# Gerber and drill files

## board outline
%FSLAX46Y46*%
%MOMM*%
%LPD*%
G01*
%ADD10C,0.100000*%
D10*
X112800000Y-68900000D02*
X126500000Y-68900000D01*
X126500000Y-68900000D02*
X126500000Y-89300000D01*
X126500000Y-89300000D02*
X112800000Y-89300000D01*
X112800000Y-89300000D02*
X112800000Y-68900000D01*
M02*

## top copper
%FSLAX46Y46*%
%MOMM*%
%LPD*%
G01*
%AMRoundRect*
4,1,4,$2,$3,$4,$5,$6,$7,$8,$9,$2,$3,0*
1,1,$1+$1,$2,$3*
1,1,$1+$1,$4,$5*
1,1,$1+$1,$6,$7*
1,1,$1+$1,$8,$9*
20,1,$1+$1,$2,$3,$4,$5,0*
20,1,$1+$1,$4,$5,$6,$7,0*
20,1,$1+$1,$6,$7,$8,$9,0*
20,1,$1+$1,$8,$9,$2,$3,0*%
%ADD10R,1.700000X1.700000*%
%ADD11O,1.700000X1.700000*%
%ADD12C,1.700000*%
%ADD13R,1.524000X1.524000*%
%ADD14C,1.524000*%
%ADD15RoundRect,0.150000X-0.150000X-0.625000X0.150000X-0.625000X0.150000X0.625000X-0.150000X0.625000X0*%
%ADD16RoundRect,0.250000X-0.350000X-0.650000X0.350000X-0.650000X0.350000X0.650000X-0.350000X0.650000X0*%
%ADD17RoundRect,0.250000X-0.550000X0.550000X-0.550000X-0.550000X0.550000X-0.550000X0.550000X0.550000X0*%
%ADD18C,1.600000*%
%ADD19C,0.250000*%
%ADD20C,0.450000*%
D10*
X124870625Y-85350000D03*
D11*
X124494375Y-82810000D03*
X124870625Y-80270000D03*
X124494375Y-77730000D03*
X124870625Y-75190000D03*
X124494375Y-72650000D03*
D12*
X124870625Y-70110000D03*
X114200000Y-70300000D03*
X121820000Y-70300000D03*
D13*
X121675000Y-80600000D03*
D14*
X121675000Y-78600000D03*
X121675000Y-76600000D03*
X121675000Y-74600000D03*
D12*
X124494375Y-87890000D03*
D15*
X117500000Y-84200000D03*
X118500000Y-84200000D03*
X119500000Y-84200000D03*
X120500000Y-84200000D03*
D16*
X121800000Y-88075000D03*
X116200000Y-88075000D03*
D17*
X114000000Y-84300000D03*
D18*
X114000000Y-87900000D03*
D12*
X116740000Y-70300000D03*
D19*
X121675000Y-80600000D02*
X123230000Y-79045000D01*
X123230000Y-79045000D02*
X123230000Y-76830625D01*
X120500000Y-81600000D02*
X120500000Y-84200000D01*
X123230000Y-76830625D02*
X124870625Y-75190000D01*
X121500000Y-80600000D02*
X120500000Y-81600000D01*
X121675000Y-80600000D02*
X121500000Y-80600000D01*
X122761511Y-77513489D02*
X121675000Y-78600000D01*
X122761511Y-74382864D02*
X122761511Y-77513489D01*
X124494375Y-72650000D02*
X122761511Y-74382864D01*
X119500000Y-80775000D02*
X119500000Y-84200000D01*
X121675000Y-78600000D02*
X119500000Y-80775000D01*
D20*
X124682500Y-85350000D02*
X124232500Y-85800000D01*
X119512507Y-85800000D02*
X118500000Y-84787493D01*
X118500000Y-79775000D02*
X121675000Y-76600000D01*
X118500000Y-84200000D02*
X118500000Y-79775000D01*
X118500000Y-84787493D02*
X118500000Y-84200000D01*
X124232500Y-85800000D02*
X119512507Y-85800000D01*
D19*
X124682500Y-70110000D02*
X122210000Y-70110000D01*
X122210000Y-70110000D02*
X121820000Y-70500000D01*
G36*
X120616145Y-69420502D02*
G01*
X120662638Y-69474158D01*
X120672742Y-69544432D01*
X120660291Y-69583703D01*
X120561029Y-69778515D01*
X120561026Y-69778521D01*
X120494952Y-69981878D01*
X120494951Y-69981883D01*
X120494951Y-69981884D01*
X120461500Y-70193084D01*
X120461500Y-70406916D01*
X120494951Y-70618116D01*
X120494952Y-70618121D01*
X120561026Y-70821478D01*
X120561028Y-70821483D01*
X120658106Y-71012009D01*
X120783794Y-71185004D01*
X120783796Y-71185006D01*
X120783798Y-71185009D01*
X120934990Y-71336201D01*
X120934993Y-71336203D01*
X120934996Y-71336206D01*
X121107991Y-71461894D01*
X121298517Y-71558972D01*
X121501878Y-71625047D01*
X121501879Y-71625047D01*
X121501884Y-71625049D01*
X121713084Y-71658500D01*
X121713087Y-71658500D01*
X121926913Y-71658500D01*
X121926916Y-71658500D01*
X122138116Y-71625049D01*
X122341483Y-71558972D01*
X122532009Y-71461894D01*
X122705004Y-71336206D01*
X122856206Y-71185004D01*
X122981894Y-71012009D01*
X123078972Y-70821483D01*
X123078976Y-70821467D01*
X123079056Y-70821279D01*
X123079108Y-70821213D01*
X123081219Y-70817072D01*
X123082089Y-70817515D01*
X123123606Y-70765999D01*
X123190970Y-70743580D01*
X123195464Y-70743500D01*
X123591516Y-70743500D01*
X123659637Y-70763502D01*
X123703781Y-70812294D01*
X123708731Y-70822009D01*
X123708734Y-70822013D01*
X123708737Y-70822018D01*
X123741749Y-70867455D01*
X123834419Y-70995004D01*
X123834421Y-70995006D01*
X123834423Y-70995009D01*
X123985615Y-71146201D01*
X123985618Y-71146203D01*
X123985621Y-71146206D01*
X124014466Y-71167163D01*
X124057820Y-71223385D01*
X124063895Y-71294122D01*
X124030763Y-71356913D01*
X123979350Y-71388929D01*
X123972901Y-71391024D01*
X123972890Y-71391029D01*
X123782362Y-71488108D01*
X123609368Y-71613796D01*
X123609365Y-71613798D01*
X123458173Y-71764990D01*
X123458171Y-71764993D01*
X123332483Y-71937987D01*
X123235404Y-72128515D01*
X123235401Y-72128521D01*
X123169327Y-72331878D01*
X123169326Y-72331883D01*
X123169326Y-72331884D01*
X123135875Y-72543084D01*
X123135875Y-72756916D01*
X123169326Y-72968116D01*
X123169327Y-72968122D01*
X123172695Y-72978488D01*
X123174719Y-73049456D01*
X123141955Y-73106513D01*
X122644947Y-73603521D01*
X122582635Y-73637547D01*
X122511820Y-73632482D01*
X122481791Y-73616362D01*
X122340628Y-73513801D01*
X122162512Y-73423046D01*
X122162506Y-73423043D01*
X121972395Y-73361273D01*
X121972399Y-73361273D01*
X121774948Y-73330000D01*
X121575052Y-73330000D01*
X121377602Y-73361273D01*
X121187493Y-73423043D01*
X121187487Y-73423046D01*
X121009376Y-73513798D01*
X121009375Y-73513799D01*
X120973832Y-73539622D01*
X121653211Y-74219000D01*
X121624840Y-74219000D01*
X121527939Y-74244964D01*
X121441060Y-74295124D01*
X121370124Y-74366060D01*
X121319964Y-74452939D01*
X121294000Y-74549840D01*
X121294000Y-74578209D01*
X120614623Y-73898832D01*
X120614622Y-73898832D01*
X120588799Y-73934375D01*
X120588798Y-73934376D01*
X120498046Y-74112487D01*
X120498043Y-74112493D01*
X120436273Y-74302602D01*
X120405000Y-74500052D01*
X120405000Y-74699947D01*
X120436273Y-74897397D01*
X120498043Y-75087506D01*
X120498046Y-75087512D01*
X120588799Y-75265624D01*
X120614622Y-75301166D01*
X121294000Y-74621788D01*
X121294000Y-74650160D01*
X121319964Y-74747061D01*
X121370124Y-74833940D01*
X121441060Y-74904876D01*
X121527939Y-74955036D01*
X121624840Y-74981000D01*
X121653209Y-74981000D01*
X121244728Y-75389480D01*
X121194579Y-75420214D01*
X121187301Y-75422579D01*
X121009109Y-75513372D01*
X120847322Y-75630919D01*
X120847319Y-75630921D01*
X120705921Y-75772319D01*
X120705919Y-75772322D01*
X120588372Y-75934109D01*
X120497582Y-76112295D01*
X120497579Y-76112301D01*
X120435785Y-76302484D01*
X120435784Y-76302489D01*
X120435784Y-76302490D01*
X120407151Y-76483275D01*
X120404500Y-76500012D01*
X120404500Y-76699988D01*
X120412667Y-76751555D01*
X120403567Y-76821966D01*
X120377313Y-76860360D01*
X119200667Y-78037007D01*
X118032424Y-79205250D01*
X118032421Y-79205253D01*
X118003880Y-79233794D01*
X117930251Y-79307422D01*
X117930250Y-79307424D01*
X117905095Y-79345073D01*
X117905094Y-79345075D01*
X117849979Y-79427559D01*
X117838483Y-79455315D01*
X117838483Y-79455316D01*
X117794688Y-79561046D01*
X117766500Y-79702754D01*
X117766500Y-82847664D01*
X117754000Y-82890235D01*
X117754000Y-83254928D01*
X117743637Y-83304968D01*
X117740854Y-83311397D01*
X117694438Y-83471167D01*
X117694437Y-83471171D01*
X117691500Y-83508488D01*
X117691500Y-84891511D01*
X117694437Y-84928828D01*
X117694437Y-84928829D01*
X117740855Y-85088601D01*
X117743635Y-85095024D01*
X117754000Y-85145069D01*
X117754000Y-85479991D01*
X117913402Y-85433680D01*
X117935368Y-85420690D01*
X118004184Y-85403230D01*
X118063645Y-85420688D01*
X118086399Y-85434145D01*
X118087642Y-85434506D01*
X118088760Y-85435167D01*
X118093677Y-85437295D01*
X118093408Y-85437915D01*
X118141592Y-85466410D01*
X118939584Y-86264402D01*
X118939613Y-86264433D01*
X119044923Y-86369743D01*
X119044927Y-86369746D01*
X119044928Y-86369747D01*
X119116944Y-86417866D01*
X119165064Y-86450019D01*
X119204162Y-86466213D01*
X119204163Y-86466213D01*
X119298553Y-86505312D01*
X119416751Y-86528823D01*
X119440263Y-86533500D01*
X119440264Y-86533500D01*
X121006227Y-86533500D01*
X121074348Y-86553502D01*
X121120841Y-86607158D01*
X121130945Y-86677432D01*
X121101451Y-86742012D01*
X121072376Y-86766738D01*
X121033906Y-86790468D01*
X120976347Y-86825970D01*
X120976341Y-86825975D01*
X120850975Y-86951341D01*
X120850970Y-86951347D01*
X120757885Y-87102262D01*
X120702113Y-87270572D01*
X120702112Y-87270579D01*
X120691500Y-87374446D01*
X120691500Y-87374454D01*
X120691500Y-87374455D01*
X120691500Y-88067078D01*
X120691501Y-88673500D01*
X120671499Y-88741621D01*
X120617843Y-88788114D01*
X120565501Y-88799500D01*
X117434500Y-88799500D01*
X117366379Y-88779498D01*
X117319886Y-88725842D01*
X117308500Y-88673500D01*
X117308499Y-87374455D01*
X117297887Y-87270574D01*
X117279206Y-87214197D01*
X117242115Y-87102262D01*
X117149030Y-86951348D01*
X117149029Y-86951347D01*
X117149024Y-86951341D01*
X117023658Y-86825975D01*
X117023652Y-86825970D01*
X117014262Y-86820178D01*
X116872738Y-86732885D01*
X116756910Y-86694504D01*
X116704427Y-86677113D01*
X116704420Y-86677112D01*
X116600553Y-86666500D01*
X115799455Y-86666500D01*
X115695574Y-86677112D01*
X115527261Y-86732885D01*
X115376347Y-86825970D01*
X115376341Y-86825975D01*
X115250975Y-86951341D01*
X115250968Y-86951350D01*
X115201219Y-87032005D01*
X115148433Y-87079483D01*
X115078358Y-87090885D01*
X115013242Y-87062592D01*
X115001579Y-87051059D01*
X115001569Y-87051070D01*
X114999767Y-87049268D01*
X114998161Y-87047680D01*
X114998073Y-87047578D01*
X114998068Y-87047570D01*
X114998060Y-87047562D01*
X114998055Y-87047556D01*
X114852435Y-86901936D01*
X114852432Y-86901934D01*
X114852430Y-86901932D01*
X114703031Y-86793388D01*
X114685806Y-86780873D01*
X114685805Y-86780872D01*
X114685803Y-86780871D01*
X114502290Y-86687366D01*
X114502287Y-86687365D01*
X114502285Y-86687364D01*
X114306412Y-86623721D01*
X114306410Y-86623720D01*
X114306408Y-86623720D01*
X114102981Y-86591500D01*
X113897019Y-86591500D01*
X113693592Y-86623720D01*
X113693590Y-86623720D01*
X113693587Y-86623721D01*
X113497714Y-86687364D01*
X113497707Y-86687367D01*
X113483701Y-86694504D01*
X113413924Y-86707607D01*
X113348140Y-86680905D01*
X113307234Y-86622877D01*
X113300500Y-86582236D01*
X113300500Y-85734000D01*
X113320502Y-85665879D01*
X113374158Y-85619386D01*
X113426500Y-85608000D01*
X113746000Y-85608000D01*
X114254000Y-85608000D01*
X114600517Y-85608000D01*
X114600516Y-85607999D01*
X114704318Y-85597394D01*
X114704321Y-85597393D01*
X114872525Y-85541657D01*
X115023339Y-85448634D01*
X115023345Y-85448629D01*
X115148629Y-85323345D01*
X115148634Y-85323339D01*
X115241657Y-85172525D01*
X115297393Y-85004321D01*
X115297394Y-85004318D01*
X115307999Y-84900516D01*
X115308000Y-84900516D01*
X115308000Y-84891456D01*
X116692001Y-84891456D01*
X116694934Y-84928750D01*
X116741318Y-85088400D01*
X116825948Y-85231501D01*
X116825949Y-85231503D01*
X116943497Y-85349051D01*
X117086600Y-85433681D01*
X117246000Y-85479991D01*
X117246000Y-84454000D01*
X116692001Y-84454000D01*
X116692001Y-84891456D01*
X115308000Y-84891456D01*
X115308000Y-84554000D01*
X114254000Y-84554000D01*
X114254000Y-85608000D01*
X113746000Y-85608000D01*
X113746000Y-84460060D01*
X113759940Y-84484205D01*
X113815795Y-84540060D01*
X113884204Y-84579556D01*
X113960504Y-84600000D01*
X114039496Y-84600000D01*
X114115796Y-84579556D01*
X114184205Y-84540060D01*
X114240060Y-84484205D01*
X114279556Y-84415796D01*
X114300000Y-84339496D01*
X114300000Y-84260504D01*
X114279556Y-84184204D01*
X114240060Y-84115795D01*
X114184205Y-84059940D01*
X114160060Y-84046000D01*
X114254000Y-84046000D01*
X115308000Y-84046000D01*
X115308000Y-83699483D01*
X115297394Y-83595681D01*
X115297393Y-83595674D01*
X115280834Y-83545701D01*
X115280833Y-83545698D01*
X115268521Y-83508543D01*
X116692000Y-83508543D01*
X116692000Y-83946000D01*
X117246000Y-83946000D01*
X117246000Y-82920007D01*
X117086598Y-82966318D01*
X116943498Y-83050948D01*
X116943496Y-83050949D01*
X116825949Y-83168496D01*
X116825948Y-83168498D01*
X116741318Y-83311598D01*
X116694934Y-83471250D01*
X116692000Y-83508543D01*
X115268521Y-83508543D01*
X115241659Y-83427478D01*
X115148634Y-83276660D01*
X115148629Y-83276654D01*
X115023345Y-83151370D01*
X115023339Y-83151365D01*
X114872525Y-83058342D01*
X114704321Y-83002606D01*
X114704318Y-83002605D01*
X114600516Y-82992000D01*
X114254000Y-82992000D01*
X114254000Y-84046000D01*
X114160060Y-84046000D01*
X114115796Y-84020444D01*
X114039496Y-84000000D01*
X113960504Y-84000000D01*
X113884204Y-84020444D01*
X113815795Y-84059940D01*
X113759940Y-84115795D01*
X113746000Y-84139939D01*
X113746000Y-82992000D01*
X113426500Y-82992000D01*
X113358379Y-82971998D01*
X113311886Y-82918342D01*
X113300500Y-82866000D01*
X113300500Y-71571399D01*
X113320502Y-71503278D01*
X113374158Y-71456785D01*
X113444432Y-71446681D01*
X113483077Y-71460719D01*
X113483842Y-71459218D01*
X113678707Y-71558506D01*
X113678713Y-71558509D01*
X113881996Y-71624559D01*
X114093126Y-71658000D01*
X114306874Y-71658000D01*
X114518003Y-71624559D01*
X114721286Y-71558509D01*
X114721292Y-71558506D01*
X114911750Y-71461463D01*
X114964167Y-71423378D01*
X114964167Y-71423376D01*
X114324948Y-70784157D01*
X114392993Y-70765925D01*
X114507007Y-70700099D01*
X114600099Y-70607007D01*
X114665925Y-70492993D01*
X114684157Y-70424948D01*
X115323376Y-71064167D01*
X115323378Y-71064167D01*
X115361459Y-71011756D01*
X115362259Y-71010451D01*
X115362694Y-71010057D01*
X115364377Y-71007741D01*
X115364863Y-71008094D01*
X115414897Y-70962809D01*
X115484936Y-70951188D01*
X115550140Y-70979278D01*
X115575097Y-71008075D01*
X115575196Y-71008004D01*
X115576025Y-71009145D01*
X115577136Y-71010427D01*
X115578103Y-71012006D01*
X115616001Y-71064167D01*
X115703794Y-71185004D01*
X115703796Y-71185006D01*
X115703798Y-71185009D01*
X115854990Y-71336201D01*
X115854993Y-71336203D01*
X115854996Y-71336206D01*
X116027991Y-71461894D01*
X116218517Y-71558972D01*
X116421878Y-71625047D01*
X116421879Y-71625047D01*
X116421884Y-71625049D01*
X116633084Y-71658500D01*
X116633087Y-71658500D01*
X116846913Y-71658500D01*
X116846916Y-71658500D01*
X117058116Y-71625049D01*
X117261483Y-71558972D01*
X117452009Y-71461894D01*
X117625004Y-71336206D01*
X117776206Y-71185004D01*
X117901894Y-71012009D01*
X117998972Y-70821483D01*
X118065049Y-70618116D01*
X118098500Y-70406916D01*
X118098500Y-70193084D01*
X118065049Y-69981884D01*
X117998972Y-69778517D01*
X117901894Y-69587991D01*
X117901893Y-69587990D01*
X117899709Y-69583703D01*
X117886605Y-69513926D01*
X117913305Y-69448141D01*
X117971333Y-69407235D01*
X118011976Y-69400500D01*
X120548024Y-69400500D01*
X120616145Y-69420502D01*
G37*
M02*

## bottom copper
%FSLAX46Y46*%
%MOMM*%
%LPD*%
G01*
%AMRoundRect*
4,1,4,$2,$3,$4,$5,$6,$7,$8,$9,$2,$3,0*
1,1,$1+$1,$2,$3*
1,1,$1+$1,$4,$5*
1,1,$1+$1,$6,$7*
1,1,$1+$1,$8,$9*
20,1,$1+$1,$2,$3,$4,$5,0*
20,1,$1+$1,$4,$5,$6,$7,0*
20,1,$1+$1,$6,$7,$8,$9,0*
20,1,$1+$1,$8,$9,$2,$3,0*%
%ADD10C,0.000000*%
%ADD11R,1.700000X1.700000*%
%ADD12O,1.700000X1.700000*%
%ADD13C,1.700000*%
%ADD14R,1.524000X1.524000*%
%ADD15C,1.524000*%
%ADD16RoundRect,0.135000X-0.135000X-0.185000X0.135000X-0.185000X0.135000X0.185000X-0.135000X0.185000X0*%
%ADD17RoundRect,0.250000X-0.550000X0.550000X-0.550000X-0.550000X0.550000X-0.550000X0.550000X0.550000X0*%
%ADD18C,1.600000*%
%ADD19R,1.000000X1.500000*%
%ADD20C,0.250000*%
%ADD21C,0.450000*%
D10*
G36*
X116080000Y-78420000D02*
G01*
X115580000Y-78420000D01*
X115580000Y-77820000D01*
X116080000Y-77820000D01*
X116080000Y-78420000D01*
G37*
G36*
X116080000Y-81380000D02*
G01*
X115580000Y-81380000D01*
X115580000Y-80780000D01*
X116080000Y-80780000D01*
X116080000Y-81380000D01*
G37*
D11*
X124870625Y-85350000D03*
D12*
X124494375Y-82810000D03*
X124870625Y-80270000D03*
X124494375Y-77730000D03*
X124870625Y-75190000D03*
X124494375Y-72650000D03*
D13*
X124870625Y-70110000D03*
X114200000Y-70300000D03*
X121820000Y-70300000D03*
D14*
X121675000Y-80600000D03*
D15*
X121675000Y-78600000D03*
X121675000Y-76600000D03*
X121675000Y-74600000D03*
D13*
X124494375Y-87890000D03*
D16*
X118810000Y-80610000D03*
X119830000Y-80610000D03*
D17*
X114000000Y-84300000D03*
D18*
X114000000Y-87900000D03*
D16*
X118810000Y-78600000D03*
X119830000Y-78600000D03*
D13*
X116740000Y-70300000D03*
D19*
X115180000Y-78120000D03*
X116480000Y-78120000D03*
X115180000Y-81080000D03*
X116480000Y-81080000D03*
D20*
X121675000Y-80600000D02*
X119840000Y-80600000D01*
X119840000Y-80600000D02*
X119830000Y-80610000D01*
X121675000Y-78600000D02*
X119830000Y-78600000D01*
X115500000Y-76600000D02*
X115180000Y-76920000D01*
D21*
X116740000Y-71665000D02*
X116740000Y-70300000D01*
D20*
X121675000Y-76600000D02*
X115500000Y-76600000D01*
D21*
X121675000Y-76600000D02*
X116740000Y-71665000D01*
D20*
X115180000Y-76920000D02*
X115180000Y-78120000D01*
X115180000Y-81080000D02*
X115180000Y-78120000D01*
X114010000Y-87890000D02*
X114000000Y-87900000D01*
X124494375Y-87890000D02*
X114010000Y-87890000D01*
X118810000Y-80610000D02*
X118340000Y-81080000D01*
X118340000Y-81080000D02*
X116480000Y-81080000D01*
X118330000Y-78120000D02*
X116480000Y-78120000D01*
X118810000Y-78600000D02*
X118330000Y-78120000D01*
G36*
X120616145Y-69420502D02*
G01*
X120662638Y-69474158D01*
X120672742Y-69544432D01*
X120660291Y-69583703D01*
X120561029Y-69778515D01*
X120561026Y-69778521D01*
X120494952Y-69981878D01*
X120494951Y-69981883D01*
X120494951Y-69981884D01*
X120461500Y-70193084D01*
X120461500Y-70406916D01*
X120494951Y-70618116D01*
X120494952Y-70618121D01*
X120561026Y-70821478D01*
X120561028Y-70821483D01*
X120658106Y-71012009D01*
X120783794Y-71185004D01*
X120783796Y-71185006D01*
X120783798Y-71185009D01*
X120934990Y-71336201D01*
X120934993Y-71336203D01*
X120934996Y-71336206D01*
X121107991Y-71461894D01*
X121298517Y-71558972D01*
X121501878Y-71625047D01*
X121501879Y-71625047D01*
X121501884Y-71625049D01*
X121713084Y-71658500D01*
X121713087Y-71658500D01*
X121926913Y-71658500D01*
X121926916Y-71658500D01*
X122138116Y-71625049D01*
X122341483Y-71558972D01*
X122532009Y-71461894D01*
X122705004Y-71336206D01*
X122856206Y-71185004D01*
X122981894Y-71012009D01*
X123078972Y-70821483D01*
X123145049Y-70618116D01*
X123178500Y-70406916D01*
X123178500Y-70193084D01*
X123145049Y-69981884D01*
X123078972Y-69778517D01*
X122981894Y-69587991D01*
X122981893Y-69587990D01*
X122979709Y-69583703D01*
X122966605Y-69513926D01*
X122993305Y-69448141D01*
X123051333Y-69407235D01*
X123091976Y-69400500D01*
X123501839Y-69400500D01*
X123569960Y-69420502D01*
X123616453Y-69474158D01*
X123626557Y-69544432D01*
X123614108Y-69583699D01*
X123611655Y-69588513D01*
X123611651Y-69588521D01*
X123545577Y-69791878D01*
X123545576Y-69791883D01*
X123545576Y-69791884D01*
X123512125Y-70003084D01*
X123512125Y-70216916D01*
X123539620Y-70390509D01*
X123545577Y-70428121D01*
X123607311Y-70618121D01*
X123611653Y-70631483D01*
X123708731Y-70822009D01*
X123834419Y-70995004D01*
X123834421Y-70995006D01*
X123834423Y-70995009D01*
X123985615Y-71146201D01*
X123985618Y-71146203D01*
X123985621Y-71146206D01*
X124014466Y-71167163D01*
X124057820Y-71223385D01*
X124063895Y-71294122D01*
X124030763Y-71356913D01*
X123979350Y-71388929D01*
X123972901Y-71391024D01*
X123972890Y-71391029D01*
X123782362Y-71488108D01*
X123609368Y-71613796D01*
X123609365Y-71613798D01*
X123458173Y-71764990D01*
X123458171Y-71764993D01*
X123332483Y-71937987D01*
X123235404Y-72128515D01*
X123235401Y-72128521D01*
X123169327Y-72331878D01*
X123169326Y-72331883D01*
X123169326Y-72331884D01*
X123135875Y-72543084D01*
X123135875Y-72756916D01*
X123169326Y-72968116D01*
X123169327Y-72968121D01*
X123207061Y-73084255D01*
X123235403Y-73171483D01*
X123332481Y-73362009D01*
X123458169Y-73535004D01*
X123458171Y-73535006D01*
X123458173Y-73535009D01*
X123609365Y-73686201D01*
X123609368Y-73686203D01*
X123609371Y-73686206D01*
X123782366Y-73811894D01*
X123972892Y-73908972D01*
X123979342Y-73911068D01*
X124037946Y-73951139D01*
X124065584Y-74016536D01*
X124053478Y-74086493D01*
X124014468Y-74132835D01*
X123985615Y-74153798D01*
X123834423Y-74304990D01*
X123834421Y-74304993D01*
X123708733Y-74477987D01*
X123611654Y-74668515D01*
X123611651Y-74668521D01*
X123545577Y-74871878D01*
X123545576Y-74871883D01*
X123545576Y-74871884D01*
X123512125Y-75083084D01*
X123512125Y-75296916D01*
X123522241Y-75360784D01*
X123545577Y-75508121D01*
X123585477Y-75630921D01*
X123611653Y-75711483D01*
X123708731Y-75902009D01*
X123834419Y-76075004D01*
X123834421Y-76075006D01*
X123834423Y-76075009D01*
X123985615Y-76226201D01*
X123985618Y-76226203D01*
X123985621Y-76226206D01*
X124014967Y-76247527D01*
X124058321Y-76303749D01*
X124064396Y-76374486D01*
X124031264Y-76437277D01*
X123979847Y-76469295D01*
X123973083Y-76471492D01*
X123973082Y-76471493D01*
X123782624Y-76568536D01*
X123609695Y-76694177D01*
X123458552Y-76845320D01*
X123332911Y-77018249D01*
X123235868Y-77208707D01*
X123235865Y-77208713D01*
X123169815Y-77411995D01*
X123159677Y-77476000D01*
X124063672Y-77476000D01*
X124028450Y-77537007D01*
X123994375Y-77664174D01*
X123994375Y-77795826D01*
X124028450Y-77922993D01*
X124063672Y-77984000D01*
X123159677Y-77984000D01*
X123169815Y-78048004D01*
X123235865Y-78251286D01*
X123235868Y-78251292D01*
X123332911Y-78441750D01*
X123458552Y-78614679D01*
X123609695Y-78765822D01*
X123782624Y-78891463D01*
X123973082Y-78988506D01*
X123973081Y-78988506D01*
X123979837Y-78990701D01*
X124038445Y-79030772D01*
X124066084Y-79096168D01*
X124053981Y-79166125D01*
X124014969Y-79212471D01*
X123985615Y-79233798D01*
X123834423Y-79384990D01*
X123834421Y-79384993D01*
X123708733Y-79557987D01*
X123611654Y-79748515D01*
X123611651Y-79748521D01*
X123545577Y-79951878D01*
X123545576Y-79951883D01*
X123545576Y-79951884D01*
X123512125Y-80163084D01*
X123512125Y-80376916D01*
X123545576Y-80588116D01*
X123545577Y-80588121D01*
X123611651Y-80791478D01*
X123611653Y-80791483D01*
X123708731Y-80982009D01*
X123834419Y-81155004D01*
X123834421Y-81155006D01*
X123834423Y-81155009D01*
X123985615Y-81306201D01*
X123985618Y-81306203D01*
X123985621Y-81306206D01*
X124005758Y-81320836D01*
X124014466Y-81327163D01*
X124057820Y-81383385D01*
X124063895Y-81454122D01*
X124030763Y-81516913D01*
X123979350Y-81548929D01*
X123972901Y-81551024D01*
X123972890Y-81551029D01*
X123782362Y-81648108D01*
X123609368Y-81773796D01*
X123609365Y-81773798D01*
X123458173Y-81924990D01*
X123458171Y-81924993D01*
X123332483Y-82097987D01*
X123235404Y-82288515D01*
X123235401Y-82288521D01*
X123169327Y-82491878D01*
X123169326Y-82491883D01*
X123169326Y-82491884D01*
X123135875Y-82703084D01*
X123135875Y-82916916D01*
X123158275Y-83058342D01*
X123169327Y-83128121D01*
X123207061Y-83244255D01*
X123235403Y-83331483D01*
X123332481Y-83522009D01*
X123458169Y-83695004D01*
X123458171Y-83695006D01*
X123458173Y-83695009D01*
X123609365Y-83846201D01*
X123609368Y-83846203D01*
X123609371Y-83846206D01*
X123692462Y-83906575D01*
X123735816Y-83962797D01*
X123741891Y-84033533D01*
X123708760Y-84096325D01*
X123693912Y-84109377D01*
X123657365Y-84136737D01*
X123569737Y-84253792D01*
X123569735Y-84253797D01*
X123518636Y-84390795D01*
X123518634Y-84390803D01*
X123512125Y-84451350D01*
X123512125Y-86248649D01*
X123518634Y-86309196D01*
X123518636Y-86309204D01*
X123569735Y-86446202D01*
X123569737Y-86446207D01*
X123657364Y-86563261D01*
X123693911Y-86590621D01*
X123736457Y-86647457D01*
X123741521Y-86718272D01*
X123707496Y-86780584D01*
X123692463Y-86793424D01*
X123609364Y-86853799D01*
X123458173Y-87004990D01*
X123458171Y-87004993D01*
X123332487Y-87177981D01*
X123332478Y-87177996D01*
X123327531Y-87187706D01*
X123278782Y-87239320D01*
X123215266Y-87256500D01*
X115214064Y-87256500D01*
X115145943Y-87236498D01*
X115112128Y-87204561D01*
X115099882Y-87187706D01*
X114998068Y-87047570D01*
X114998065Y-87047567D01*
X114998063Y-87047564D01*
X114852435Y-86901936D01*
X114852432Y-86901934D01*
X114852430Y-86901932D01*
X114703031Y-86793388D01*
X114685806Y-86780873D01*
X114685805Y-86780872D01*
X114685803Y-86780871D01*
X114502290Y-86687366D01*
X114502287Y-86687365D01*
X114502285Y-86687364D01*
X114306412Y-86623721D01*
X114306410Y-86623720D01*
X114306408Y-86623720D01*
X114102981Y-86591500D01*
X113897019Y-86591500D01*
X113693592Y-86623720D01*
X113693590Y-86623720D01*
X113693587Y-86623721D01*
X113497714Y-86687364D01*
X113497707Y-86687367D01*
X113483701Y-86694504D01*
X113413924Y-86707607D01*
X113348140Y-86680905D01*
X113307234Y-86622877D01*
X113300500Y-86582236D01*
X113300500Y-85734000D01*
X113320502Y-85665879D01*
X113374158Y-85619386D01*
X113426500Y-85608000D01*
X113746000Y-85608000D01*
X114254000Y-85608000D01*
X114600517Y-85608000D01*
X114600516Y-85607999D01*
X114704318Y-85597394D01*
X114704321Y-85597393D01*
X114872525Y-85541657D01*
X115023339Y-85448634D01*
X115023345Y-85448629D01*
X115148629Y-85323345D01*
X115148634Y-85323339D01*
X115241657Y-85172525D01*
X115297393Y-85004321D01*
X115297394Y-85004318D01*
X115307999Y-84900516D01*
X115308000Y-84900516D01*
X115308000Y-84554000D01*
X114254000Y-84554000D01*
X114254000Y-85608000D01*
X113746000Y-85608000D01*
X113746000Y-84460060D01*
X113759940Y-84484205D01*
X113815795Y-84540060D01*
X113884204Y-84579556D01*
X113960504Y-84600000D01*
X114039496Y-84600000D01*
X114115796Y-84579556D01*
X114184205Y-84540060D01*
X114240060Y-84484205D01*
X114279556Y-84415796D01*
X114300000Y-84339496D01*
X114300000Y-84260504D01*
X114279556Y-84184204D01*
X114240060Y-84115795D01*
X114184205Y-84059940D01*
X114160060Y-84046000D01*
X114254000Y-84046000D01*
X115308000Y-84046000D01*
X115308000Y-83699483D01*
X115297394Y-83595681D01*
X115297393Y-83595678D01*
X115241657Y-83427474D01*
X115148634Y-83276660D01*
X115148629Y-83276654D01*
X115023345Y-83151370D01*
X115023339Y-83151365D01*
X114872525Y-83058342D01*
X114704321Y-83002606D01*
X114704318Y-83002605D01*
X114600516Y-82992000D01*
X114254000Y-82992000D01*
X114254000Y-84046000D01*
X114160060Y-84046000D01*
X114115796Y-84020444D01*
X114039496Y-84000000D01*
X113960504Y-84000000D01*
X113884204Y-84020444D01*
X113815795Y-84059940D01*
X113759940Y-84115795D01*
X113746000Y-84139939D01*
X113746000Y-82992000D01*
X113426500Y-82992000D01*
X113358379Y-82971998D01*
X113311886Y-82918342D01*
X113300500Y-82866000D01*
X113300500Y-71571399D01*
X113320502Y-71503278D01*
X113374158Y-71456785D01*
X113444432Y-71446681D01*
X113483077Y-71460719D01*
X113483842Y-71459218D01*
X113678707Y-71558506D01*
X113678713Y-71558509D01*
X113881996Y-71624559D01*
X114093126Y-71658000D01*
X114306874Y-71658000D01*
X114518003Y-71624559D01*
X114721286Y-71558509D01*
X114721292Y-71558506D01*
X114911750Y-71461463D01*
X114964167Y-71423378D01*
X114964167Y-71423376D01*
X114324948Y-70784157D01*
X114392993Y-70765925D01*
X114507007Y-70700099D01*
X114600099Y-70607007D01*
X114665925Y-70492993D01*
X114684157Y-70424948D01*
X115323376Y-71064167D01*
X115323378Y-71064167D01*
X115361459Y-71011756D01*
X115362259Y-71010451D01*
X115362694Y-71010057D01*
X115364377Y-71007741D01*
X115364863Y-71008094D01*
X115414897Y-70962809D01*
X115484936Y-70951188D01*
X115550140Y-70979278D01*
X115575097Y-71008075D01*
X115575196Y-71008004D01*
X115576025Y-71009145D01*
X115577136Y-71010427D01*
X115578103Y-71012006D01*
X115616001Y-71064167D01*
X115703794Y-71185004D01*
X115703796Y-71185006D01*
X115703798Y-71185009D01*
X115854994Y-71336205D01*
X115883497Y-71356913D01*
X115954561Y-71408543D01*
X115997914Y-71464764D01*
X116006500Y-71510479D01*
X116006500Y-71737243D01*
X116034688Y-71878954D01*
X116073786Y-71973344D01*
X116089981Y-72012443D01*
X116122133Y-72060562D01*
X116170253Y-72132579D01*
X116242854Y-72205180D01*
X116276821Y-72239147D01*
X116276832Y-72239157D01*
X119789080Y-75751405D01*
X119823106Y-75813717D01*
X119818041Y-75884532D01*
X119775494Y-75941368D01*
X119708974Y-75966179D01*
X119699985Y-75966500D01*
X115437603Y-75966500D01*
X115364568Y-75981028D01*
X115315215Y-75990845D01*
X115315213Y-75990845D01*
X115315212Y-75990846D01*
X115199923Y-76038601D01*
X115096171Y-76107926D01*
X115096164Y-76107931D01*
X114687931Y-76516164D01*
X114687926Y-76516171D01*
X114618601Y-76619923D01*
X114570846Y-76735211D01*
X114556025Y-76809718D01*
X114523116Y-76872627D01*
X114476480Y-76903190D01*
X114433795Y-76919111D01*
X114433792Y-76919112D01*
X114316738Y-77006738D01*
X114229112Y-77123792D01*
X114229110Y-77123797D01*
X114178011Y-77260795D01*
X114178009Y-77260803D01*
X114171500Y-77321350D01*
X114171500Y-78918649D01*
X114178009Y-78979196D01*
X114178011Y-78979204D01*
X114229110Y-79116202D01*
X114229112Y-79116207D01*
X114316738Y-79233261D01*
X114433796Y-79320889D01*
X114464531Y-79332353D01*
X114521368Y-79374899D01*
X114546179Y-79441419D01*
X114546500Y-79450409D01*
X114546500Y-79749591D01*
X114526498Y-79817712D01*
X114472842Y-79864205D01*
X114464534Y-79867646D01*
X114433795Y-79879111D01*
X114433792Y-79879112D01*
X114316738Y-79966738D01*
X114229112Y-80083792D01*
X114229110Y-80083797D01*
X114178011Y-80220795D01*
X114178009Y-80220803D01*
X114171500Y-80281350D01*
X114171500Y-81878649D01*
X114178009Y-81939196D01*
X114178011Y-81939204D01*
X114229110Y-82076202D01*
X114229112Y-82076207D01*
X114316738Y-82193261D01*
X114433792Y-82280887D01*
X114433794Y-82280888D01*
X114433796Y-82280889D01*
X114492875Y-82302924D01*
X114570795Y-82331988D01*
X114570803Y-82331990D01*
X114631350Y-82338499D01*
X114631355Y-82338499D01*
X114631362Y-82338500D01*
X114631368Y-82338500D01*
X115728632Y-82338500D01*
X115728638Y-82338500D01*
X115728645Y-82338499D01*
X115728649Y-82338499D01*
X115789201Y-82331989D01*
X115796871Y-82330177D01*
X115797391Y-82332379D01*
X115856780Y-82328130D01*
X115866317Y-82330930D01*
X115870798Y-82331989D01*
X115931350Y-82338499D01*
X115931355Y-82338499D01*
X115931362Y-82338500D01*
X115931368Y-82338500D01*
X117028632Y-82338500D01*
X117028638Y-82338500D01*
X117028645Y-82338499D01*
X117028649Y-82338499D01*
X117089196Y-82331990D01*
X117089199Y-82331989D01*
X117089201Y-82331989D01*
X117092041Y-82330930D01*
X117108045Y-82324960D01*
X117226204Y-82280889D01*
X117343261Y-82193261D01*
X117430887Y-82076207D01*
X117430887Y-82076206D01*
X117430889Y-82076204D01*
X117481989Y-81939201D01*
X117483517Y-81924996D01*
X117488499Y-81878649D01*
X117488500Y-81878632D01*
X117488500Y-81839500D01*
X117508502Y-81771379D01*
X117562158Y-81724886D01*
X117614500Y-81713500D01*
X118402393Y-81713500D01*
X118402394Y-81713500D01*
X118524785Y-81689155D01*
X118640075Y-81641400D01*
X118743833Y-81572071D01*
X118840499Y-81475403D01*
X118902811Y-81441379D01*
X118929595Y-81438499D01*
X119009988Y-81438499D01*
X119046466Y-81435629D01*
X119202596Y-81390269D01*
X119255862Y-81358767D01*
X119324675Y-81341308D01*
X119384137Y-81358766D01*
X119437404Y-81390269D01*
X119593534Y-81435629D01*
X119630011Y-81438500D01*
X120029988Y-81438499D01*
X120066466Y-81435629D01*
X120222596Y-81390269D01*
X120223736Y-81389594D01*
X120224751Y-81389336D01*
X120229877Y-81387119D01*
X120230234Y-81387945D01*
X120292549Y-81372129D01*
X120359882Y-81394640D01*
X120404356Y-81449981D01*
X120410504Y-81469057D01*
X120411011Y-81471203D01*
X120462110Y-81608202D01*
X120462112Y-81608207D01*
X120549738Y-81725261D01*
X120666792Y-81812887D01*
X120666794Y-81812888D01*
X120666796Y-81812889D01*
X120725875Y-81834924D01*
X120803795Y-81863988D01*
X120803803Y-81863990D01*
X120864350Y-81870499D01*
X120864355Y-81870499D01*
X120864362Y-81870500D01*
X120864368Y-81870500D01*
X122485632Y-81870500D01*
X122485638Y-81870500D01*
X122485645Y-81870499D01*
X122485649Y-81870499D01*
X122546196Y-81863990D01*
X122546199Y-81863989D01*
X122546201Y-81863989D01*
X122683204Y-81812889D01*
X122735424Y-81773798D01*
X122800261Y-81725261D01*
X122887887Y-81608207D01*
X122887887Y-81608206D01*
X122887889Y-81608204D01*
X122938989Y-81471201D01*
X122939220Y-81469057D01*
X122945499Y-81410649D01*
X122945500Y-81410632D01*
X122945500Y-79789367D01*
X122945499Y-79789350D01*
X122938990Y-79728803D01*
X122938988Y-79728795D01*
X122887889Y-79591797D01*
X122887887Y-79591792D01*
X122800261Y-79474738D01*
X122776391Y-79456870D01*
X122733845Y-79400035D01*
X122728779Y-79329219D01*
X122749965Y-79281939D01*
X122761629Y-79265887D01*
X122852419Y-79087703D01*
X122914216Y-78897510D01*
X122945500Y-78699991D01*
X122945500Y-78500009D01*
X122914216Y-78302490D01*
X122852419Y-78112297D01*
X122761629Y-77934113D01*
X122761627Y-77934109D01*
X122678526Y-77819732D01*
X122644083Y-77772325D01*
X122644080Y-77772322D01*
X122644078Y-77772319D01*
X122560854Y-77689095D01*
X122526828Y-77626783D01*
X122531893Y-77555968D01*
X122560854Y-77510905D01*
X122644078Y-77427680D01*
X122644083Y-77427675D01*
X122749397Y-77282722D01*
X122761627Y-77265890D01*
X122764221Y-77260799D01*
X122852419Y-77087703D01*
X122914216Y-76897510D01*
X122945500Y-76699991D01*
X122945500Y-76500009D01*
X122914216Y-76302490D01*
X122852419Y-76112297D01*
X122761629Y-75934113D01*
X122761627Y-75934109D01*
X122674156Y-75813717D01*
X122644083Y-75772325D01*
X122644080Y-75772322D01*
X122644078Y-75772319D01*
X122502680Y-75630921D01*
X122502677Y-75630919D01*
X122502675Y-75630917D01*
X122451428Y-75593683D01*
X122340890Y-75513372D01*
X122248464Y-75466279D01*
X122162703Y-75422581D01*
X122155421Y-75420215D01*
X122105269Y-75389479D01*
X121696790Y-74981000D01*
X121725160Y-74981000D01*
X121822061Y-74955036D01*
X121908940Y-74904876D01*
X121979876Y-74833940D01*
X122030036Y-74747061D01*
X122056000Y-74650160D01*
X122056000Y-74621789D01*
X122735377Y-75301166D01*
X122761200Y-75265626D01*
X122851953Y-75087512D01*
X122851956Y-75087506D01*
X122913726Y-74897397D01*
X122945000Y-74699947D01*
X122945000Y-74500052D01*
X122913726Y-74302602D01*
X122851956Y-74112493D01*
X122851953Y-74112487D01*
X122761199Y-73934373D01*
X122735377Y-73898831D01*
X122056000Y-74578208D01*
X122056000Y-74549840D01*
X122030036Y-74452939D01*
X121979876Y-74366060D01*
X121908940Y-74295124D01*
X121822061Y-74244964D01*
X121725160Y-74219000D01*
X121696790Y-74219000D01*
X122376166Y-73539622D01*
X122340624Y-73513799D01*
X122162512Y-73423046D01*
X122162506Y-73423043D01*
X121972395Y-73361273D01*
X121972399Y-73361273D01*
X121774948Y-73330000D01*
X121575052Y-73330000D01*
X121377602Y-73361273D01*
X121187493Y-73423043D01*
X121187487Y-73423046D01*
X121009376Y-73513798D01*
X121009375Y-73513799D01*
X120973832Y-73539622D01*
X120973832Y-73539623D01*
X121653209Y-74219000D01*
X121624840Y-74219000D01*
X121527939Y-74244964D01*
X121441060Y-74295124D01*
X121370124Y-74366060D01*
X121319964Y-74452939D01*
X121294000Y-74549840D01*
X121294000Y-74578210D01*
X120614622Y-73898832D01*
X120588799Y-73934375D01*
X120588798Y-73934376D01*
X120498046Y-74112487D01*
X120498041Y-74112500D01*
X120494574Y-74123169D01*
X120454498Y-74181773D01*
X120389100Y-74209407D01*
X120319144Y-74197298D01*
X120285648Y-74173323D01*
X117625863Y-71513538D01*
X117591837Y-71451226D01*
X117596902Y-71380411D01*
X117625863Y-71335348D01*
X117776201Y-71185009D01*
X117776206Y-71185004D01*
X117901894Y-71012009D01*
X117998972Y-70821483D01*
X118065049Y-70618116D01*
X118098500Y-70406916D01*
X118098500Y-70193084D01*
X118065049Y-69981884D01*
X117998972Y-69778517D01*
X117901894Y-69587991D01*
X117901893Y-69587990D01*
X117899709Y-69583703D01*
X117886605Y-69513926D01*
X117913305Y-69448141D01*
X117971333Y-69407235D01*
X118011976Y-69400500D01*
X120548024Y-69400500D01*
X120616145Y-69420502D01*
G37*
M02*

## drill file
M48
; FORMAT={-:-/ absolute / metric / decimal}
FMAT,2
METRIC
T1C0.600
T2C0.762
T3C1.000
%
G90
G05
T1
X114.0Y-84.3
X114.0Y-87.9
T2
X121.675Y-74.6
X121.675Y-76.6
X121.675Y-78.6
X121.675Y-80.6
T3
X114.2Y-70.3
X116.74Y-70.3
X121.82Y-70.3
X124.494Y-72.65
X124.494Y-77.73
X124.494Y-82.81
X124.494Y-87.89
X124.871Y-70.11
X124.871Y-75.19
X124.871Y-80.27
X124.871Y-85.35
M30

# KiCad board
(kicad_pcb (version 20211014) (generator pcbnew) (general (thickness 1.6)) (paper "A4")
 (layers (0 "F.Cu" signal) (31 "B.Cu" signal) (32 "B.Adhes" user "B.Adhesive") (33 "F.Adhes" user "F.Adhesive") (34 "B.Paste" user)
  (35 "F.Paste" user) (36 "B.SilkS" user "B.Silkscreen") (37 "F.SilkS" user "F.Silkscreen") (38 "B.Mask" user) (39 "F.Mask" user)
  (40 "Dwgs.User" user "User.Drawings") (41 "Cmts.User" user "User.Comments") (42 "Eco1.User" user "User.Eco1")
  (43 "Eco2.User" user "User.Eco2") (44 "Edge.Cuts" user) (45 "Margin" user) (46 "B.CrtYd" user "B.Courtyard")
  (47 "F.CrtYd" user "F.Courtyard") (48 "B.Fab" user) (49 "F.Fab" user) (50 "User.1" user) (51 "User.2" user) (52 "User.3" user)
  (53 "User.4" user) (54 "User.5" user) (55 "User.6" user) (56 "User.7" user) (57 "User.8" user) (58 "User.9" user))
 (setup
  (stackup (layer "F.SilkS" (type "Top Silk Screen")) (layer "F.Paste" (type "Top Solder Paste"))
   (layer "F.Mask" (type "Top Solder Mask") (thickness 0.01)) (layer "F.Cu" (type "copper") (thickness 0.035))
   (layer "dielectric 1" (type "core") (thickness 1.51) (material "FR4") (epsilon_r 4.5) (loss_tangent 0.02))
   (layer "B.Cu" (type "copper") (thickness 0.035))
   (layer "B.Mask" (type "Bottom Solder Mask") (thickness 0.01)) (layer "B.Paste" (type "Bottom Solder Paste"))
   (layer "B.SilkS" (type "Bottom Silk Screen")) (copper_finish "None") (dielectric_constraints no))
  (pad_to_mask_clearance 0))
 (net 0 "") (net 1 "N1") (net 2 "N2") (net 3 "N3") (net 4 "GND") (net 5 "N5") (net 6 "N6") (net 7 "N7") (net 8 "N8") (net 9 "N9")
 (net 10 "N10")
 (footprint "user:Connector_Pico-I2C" (layer "F.Cu") (at 124.870625 85.35 180)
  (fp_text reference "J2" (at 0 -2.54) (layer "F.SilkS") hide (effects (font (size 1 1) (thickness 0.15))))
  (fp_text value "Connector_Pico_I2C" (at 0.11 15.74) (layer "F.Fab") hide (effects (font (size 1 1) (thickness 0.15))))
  (pad "1" thru_hole rect (at 0 0 180) (size 1.7 1.7) (drill 1) (layers *.Cu *.Mask) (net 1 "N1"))
  (pad "2" thru_hole oval (at 0.37625 2.54 180) (size 1.7 1.7) (drill 1) (layers *.Cu *.Mask) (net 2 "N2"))
  (pad "3" thru_hole oval (at 0 5.08 180) (size 1.7 1.7) (drill 1) (layers *.Cu *.Mask) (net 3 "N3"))
  (pad "4" thru_hole oval (at 0.37625 7.62 180) (size 1.7 1.7) (drill 1) (layers *.Cu *.Mask) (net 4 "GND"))
  (pad "5" thru_hole oval (at 0 10.16 180) (size 1.7 1.7) (drill 1) (layers *.Cu *.Mask) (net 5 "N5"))
  (pad "6" thru_hole oval (at 0.37625 12.7 180) (size 1.7 1.7) (drill 1) (layers *.Cu *.Mask) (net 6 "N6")))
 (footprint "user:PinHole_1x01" (layer "F.Cu") (at 124.870625 70.11)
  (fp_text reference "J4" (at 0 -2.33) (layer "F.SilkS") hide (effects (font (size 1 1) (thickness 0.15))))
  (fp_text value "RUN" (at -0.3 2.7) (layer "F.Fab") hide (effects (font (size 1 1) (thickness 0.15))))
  (pad "1" thru_hole circle (at 0 0) (size 1.7 1.7) (drill 1) (layers *.Cu *.Mask) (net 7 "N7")))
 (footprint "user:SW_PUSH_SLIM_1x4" (layer "F.Cu") (at 114.2 70.3)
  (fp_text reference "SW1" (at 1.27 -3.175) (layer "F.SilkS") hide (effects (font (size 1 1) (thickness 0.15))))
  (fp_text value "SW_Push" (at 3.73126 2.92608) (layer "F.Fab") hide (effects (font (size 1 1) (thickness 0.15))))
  (pad "1" thru_hole circle locked (at 0 0) (size 1.7 1.7) (drill 1) (layers *.Cu *.Mask) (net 4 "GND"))
  (pad "2" thru_hole circle locked (at 7.62 0) (size 1.7 1.7) (drill 1) (layers *.Cu *.Mask) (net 7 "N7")))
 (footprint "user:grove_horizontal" (layer "F.Cu") (at 121.675 77.6 -90)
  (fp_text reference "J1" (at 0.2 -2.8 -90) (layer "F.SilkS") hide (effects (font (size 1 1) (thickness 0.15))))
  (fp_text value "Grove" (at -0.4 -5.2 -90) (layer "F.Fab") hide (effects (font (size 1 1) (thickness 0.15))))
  (pad "1" thru_hole rect (at 3 0 270) (size 1.524 1.524) (drill 0.762) (layers *.Cu *.Mask) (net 5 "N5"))
  (pad "2" thru_hole circle (at 1 0 270) (size 1.524 1.524) (drill 0.762) (layers *.Cu *.Mask) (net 6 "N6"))
  (pad "3" thru_hole circle (at -1 0 270) (size 1.524 1.524) (drill 0.762) (layers *.Cu *.Mask) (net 1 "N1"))
  (pad "4" thru_hole circle (at -3 0 270) (size 1.524 1.524) (drill 0.762) (layers *.Cu *.Mask) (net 4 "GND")))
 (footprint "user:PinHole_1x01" (layer "F.Cu") (at 124.494375 87.89)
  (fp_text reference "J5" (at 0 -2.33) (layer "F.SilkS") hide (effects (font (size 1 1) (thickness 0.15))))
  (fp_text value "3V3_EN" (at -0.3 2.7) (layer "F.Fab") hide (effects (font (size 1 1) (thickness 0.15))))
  (pad "1" thru_hole circle (at 0 0) (size 1.7 1.7) (drill 1) (layers *.Cu *.Mask) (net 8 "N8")))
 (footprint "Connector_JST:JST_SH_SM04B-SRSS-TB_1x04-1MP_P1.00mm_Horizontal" (layer "F.Cu") (at 119 86.2)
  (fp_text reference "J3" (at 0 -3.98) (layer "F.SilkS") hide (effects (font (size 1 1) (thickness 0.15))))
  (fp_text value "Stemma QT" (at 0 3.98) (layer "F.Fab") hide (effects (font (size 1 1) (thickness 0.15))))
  (pad "1" smd roundrect (at -1.5 -2) (size 0.6 1.55) (layers "F.Cu" "F.Paste" "F.Mask") (roundrect_rratio 0.25) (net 4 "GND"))
  (pad "2" smd roundrect (at -0.5 -2) (size 0.6 1.55) (layers "F.Cu" "F.Paste" "F.Mask") (roundrect_rratio 0.25) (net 1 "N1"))
  (pad "3" smd roundrect (at 0.5 -2) (size 0.6 1.55) (layers "F.Cu" "F.Paste" "F.Mask") (roundrect_rratio 0.25) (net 6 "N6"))
  (pad "4" smd roundrect (at 1.5 -2) (size 0.6 1.55) (layers "F.Cu" "F.Paste" "F.Mask") (roundrect_rratio 0.25) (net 5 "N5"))
  (pad "MP" smd roundrect (at 2.8 1.875) (size 1.2 1.8) (layers "F.Cu" "F.Paste" "F.Mask") (roundrect_rratio 0.2083333333))
  (pad "MP" smd roundrect (at -2.8 1.875) (size 1.2 1.8) (layers "F.Cu" "F.Paste" "F.Mask") (roundrect_rratio 0.2083333333)))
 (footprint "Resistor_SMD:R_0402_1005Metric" (layer "B.Cu") (at 119.32 80.61)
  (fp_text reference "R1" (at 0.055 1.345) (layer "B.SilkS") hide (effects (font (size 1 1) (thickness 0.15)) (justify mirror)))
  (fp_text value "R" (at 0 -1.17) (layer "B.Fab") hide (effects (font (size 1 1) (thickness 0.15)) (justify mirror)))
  (pad "1" smd roundrect (at -0.51 0) (size 0.54 0.64) (layers "B.Cu" "B.Paste" "B.Mask") (roundrect_rratio 0.25) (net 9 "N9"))
  (pad "2" smd roundrect (at 0.51 0) (size 0.54 0.64) (layers "B.Cu" "B.Paste" "B.Mask") (roundrect_rratio 0.25) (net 5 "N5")))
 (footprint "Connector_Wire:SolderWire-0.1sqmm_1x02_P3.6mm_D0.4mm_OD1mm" (layer "B.Cu") (at 114 84.3 -90)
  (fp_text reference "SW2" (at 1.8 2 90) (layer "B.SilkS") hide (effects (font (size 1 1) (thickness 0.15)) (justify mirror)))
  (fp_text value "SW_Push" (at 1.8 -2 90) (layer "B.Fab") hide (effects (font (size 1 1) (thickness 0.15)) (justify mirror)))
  (pad "1" thru_hole roundrect (at 0 0 270) (size 1.6 1.6) (drill 0.6) (layers *.Cu *.Mask) (roundrect_rratio 0.15625) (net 4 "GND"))
  (pad "2" thru_hole circle (at 3.6 0 270) (size 1.6 1.6) (drill 0.6) (layers *.Cu *.Mask) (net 8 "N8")))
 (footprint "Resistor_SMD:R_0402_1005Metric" (layer "B.Cu") (at 119.32 78.6)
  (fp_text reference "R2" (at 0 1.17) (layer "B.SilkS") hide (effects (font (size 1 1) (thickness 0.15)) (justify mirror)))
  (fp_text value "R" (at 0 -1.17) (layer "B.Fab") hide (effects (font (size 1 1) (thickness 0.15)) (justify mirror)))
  (pad "1" smd roundrect (at -0.51 0) (size 0.54 0.64) (layers "B.Cu" "B.Paste" "B.Mask") (roundrect_rratio 0.25) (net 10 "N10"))
  (pad "2" smd roundrect (at 0.51 0) (size 0.54 0.64) (layers "B.Cu" "B.Paste" "B.Mask") (roundrect_rratio 0.25) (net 6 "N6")))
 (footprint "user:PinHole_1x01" (layer "B.Cu") (at 116.81 70.3 180)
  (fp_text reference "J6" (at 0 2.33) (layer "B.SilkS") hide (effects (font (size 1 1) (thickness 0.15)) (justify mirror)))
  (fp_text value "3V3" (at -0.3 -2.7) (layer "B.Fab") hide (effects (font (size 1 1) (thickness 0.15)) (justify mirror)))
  (pad "1" thru_hole circle (at 0.07 0 180) (size 1.7 1.7) (drill 1) (layers *.Cu *.Mask) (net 1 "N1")))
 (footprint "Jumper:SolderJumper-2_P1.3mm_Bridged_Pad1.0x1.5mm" (layer "B.Cu") (at 115.83 78.12)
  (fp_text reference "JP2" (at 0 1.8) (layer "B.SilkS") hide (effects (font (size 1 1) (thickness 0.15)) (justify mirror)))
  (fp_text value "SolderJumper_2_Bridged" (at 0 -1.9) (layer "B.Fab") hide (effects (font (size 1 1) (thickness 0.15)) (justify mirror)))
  (fp_poly (pts (xy -0.25 0.3) (xy 0.25 0.3) (xy 0.25 -0.3) (xy -0.25 -0.3)) (layer "B.Cu") (width 0) (fill solid))
  (pad "1" smd rect (at -0.65 0) (size 1 1.5) (layers "B.Cu" "B.Mask") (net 1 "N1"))
  (pad "2" smd rect (at 0.65 0) (size 1 1.5) (layers "B.Cu" "B.Mask") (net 10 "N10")))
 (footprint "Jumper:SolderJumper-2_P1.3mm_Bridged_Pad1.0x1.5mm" (layer "B.Cu") (at 115.83 81.08)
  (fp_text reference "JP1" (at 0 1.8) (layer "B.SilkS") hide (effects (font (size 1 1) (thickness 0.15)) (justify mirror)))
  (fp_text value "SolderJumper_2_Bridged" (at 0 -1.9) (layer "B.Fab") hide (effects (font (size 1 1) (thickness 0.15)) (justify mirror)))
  (fp_poly (pts (xy -0.25 0.3) (xy 0.25 0.3) (xy 0.25 -0.3) (xy -0.25 -0.3)) (layer "B.Cu") (width 0) (fill solid))
  (pad "1" smd rect (at -0.65 0) (size 1 1.5) (layers "B.Cu" "B.Mask") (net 1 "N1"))
  (pad "2" smd rect (at 0.65 0) (size 1 1.5) (layers "B.Cu" "B.Mask") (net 9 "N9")))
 (gr_line (start 112.8 68.9) (end 126.5 68.9) (layer "Edge.Cuts") (width 0.1))
 (gr_line (start 126.5 68.9) (end 126.5 89.3) (layer "Edge.Cuts") (width 0.1))
 (gr_line (start 126.5 89.3) (end 112.8 89.3) (layer "Edge.Cuts") (width 0.1))
 (gr_line (start 112.8 89.3) (end 112.8 68.9) (layer "Edge.Cuts") (width 0.1))
 (segment (start 121.675 80.6) (end 123.23 79.045) (width 0.25) (layer "F.Cu") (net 5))
 (segment (start 123.23 79.045) (end 123.23 76.830625) (width 0.25) (layer "F.Cu") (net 5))
 (segment (start 120.5 81.6) (end 120.5 84.2) (width 0.25) (layer "F.Cu") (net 5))
 (segment (start 123.23 76.830625) (end 124.870625 75.19) (width 0.25) (layer "F.Cu") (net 5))
 (segment (start 121.5 80.6) (end 120.5 81.6) (width 0.25) (layer "F.Cu") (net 5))
 (segment (start 121.675 80.6) (end 121.5 80.6) (width 0.25) (layer "F.Cu") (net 5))
 (segment (start 121.675 80.6) (end 119.84 80.6) (width 0.25) (layer "B.Cu") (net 5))
 (segment (start 119.84 80.6) (end 119.83 80.61) (width 0.25) (layer "B.Cu") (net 5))
 (segment (start 122.761511 77.513489) (end 121.675 78.6) (width 0.25) (layer "F.Cu") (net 6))
 (segment (start 122.761511 74.382864) (end 122.761511 77.513489) (width 0.25) (layer "F.Cu") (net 6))
 (segment (start 124.494375 72.65) (end 122.761511 74.382864) (width 0.25) (layer "F.Cu") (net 6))
 (segment (start 119.5 80.775) (end 119.5 84.2) (width 0.25) (layer "F.Cu") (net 6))
 (segment (start 121.675 78.6) (end 119.5 80.775) (width 0.25) (layer "F.Cu") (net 6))
 (segment (start 121.675 78.6) (end 119.83 78.6) (width 0.25) (layer "B.Cu") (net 6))
 (segment (start 124.6825 85.35) (end 124.2325 85.8) (width 0.45) (layer "F.Cu") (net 1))
 (segment (start 119.512507 85.8) (end 118.5 84.787493) (width 0.45) (layer "F.Cu") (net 1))
 (segment (start 118.5 79.775) (end 121.675 76.6) (width 0.45) (layer "F.Cu") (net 1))
 (segment (start 118.5 84.2) (end 118.5 79.775) (width 0.45) (layer "F.Cu") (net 1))
 (segment (start 118.5 84.787493) (end 118.5 84.2) (width 0.45) (layer "F.Cu") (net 1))
 (segment (start 124.2325 85.8) (end 119.512507 85.8) (width 0.45) (layer "F.Cu") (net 1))
 (segment (start 115.5 76.6) (end 115.18 76.92) (width 0.25) (layer "B.Cu") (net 1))
 (segment (start 116.74 71.665) (end 116.74 70.3) (width 0.45) (layer "B.Cu") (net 1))
 (segment (start 121.675 76.6) (end 115.5 76.6) (width 0.25) (layer "B.Cu") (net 1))
 (segment (start 121.675 76.6) (end 116.74 71.665) (width 0.45) (layer "B.Cu") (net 1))
 (segment (start 115.18 76.92) (end 115.18 78.12) (width 0.25) (layer "B.Cu") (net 1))
 (segment (start 115.18 81.08) (end 115.18 78.12) (width 0.25) (layer "B.Cu") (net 1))
 (segment (start 114.01 87.89) (end 114 87.9) (width 0.25) (layer "B.Cu") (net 8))
 (segment (start 124.494375 87.89) (end 114.01 87.89) (width 0.25) (layer "B.Cu") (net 8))
 (segment (start 124.6825 70.11) (end 122.21 70.11) (width 0.25) (layer "F.Cu") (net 7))
 (segment (start 122.21 70.11) (end 121.82 70.5) (width 0.25) (layer "F.Cu") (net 7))
 (segment (start 118.81 80.61) (end 118.34 81.08) (width 0.25) (layer "B.Cu") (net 9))
 (segment (start 118.34 81.08) (end 116.48 81.08) (width 0.25) (layer "B.Cu") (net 9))
 (segment (start 118.33 78.12) (end 116.48 78.12) (width 0.25) (layer "B.Cu") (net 10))
 (segment (start 118.81 78.6) (end 118.33 78.12) (width 0.25) (layer "B.Cu") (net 10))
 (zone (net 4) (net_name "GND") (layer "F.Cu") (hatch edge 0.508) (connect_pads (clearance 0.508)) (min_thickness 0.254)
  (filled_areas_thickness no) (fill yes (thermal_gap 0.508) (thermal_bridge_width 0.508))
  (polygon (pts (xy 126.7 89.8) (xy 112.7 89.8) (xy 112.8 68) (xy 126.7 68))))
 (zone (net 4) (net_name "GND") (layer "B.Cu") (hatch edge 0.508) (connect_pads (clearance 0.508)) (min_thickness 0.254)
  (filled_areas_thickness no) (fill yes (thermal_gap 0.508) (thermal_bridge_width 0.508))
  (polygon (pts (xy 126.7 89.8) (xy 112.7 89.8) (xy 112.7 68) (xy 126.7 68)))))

